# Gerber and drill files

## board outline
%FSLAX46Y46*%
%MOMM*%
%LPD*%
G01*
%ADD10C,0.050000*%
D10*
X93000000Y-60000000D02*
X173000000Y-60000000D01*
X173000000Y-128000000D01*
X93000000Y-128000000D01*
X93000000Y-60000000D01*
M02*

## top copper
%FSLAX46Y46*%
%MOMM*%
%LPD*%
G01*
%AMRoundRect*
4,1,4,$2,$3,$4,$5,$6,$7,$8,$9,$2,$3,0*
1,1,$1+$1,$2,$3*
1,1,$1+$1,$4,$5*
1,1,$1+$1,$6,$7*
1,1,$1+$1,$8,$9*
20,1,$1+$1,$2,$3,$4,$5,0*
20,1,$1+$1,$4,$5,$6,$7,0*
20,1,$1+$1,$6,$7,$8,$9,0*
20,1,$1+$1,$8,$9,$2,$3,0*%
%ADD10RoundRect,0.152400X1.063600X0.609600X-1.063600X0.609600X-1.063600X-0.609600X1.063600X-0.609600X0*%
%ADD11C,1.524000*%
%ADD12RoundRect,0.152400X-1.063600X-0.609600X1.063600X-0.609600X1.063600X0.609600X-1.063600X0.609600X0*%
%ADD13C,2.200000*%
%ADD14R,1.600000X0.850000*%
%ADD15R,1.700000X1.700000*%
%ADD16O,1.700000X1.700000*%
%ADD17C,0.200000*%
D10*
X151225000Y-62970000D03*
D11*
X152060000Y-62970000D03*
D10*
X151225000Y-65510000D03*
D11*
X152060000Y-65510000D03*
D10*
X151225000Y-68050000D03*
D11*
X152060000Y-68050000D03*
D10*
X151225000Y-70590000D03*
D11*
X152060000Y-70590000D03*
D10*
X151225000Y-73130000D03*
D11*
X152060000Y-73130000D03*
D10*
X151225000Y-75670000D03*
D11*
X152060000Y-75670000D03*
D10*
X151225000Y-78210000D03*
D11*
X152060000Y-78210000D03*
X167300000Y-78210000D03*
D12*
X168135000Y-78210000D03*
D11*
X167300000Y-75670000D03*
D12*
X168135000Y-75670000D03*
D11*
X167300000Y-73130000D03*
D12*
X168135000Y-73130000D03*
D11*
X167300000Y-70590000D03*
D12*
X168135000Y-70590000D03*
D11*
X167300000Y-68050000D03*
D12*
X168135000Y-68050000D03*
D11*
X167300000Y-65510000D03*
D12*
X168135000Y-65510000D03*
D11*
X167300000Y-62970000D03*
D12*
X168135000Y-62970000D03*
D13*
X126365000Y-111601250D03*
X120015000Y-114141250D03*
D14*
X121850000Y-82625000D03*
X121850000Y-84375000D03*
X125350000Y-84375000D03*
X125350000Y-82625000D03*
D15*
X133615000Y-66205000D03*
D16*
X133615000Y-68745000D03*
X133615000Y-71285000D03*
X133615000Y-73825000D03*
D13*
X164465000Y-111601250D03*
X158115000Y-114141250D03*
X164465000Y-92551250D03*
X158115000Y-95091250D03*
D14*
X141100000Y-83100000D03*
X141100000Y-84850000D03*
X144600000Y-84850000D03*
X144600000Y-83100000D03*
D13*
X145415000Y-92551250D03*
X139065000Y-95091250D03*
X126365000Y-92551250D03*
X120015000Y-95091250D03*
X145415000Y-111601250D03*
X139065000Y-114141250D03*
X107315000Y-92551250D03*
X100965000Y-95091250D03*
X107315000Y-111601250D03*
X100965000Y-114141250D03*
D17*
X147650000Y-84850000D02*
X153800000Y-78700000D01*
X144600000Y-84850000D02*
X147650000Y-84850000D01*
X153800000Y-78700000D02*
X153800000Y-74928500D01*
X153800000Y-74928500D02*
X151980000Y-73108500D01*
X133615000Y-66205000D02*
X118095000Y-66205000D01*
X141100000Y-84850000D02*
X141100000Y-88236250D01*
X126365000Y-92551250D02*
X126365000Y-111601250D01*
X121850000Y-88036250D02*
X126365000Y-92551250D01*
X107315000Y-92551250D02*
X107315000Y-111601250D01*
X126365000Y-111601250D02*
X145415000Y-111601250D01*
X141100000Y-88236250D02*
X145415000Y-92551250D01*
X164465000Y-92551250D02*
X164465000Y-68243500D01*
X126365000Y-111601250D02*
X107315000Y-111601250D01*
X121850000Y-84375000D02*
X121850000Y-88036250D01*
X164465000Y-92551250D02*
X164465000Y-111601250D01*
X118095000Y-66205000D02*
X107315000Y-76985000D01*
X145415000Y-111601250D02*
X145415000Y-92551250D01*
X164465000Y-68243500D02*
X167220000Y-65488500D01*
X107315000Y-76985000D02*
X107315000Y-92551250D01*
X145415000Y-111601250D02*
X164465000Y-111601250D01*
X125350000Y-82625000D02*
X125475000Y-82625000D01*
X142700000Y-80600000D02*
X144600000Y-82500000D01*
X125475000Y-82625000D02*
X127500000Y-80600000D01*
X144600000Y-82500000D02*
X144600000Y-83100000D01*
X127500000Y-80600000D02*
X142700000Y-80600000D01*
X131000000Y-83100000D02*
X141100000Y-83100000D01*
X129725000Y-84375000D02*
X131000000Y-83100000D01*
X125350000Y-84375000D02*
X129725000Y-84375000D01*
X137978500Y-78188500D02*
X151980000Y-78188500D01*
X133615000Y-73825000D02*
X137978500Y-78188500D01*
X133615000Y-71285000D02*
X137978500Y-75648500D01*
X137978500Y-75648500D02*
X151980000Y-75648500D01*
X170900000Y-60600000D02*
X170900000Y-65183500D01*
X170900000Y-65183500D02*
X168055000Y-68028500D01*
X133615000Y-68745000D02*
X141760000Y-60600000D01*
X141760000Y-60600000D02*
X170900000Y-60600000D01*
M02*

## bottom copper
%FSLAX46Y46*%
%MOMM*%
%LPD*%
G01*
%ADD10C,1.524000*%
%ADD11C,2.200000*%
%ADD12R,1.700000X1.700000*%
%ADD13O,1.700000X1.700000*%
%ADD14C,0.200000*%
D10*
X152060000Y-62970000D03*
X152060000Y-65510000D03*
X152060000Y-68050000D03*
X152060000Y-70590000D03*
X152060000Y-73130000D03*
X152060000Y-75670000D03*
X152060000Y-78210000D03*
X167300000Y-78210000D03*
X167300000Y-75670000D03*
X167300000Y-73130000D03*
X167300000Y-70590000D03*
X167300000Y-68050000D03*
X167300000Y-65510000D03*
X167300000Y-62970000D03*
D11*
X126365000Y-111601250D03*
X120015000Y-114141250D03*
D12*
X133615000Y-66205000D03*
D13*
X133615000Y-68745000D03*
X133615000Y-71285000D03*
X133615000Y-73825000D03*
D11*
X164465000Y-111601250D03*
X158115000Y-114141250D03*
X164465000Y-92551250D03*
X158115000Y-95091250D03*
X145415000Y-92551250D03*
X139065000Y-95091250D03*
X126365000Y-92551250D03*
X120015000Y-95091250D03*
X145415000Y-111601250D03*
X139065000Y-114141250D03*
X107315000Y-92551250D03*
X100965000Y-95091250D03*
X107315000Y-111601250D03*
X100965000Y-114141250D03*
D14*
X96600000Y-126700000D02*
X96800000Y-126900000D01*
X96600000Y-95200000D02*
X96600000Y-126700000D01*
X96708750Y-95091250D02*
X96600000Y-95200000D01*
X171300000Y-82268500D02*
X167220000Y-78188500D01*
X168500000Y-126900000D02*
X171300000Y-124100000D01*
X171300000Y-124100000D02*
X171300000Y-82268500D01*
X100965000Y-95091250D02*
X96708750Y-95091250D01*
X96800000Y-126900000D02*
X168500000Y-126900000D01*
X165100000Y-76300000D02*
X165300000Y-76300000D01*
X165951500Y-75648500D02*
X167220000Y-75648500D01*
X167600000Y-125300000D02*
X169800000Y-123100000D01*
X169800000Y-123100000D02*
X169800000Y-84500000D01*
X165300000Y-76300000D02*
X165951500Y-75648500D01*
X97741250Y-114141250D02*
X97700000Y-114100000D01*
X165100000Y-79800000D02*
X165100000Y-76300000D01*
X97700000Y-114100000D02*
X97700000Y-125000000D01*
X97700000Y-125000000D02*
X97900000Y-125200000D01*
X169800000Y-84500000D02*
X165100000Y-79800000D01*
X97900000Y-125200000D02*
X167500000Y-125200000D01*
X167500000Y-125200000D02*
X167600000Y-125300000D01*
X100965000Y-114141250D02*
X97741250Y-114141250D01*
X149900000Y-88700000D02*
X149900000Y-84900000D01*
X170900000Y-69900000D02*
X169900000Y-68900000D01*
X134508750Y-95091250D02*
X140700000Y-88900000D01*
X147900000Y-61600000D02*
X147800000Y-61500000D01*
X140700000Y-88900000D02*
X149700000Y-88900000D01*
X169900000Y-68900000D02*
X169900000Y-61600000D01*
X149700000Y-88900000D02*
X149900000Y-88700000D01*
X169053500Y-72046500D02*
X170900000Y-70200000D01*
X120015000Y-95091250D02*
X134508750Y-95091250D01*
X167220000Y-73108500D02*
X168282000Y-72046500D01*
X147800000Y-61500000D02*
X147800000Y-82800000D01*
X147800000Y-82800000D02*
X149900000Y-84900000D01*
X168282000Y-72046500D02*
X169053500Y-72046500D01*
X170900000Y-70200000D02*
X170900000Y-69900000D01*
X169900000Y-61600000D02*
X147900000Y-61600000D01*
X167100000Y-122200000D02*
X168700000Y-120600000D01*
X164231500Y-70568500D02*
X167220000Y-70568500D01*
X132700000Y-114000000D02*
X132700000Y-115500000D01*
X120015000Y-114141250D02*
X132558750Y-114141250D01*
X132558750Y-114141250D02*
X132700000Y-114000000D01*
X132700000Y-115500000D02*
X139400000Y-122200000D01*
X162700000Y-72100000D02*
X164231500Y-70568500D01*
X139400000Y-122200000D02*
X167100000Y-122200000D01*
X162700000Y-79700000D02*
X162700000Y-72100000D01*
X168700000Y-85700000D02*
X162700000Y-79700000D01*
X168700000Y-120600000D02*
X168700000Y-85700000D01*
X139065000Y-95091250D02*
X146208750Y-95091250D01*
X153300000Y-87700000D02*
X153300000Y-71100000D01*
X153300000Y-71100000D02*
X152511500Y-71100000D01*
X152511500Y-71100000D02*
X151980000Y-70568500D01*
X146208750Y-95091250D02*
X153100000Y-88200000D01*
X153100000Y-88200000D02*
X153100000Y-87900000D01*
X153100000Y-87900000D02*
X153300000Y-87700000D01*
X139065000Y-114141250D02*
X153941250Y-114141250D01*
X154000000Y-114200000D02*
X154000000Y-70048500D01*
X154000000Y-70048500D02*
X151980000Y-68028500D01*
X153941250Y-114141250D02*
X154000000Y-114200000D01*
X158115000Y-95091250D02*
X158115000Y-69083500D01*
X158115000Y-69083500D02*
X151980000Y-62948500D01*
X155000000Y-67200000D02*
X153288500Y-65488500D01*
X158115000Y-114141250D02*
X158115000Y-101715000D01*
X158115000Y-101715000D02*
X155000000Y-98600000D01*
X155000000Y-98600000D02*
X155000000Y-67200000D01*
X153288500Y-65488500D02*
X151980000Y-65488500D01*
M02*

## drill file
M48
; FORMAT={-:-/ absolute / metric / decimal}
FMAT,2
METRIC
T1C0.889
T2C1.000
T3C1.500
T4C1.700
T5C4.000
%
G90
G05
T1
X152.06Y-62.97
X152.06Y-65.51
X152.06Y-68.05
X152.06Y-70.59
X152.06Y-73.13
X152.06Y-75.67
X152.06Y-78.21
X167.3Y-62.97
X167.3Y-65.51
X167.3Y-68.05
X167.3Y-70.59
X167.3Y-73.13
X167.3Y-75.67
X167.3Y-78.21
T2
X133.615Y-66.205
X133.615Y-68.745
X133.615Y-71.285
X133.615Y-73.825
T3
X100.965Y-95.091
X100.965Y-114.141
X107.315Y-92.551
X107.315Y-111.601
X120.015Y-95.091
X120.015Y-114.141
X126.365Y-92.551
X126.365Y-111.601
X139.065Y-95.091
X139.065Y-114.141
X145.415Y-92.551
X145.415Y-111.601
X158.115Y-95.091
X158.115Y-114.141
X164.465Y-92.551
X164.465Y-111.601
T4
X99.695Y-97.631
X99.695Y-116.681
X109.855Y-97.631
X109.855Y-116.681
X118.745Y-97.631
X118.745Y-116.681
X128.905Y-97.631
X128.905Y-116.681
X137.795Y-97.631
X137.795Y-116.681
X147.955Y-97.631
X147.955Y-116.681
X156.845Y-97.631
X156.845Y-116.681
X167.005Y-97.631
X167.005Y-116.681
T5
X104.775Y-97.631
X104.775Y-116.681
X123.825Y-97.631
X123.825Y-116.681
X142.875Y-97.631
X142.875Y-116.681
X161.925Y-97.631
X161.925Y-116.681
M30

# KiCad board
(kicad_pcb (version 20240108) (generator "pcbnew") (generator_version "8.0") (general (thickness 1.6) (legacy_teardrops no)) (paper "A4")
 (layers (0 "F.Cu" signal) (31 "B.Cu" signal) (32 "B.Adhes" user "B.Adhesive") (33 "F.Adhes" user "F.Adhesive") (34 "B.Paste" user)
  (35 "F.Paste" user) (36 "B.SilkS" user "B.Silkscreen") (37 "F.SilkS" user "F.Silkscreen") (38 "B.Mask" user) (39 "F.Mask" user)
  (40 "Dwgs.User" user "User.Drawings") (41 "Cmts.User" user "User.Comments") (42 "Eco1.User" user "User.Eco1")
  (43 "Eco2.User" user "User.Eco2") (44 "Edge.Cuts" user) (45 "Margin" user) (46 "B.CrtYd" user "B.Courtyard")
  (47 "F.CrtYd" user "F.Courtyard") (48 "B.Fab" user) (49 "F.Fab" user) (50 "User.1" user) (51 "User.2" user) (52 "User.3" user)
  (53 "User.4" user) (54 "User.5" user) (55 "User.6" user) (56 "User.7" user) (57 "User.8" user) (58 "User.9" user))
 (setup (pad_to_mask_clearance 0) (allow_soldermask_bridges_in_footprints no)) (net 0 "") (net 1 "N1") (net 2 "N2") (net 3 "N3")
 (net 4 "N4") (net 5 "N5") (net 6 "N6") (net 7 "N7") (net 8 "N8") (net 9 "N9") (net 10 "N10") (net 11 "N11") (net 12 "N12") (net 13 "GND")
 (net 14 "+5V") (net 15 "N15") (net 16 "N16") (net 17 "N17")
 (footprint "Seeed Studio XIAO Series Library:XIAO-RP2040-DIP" (layer "F.Cu") (at 159.68 70.59)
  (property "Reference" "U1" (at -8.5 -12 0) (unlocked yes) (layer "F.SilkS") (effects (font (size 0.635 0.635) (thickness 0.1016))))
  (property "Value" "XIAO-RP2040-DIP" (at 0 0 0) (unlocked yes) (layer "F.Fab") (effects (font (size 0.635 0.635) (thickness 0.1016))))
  (pad "1" smd roundrect (at -8.455 -7.62 180) (size 2.432 1.524) (layers "F.Cu" "F.Mask") (roundrect_rratio 0.1) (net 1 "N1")
   (thermal_bridge_angle 45))
  (pad "1" thru_hole circle (at -7.62 -7.62 180) (size 1.524 1.524) (drill 0.889) (layers "*.Cu" "*.Mask") (remove_unused_layers no)
   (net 1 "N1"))
  (pad "2" smd roundrect (at -8.455 -5.08 180) (size 2.432 1.524) (layers "F.Cu" "F.Mask") (roundrect_rratio 0.1) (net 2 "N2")
   (thermal_bridge_angle 45))
  (pad "2" thru_hole circle (at -7.62 -5.08 180) (size 1.524 1.524) (drill 0.889) (layers "*.Cu" "*.Mask") (remove_unused_layers no)
   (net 2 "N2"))
  (pad "3" smd roundrect (at -8.455 -2.54 180) (size 2.432 1.524) (layers "F.Cu" "F.Mask") (roundrect_rratio 0.1) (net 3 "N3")
   (thermal_bridge_angle 45))
  (pad "3" thru_hole circle (at -7.62 -2.54 180) (size 1.524 1.524) (drill 0.889) (layers "*.Cu" "*.Mask") (remove_unused_layers no)
   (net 3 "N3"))
  (pad "4" smd roundrect (at -8.455 0 180) (size 2.432 1.524) (layers "F.Cu" "F.Mask") (roundrect_rratio 0.1) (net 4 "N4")
   (thermal_bridge_angle 45))
  (pad "4" thru_hole circle (at -7.62 0 180) (size 1.524 1.524) (drill 0.889) (layers "*.Cu" "*.Mask") (remove_unused_layers no)
   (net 4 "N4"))
  (pad "5" smd roundrect (at -8.455 2.54 180) (size 2.432 1.524) (layers "F.Cu" "F.Mask") (roundrect_rratio 0.1) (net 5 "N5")
   (thermal_bridge_angle 45))
  (pad "5" thru_hole circle (at -7.62 2.54 180) (size 1.524 1.524) (drill 0.889) (layers "*.Cu" "*.Mask") (remove_unused_layers no)
   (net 5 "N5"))
  (pad "6" smd roundrect (at -8.455 5.08 180) (size 2.432 1.524) (layers "F.Cu" "F.Mask") (roundrect_rratio 0.1) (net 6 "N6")
   (thermal_bridge_angle 45))
  (pad "6" thru_hole circle (at -7.62 5.08 180) (size 1.524 1.524) (drill 0.889) (layers "*.Cu" "*.Mask") (remove_unused_layers no)
   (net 6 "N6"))
  (pad "7" smd roundrect (at -8.455 7.62 180) (size 2.432 1.524) (layers "F.Cu" "F.Mask") (roundrect_rratio 0.1) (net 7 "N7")
   (thermal_bridge_angle 45))
  (pad "7" thru_hole circle (at -7.62 7.62 180) (size 1.524 1.524) (drill 0.889) (layers "*.Cu" "*.Mask") (remove_unused_layers no)
   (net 7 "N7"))
  (pad "8" thru_hole circle (at 7.62 7.62) (size 1.524 1.524) (drill 0.889) (layers "*.Cu" "*.Mask") (remove_unused_layers no) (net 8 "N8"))
  (pad "8" smd roundrect (at 8.455 7.62) (size 2.432 1.524) (layers "F.Cu" "F.Mask") (roundrect_rratio 0.1) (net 8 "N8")
   (thermal_bridge_angle 45))
  (pad "9" thru_hole circle (at 7.62 5.08) (size 1.524 1.524) (drill 0.889) (layers "*.Cu" "*.Mask") (remove_unused_layers no) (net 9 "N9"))
  (pad "9" smd roundrect (at 8.455 5.08) (size 2.432 1.524) (layers "F.Cu" "F.Mask") (roundrect_rratio 0.1) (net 9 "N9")
   (thermal_bridge_angle 45))
  (pad "10" thru_hole circle (at 7.62 2.54) (size 1.524 1.524) (drill 0.889) (layers "*.Cu" "*.Mask") (remove_unused_layers no)
   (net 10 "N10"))
  (pad "10" smd roundrect (at 8.455 2.54) (size 2.432 1.524) (layers "F.Cu" "F.Mask") (roundrect_rratio 0.1) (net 10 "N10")
   (thermal_bridge_angle 45))
  (pad "11" thru_hole circle (at 7.62 0) (size 1.524 1.524) (drill 0.889) (layers "*.Cu" "*.Mask") (remove_unused_layers no) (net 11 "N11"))
  (pad "11" smd roundrect (at 8.455 0) (size 2.432 1.524) (layers "F.Cu" "F.Mask") (roundrect_rratio 0.1) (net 11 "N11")
   (thermal_bridge_angle 45))
  (pad "12" thru_hole circle (at 7.62 -2.54) (size 1.524 1.524) (drill 0.889) (layers "*.Cu" "*.Mask") (remove_unused_layers no)
   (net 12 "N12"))
  (pad "12" smd roundrect (at 8.455 -2.54) (size 2.432 1.524) (layers "F.Cu" "F.Mask") (roundrect_rratio 0.1) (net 12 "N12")
   (thermal_bridge_angle 45))
  (pad "13" thru_hole circle (at 7.62 -5.08) (size 1.524 1.524) (drill 0.889) (layers "*.Cu" "*.Mask") (remove_unused_layers no)
   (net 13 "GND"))
  (pad "13" smd roundrect (at 8.455 -5.08) (size 2.432 1.524) (layers "F.Cu" "F.Mask") (roundrect_rratio 0.1) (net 13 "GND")
   (thermal_bridge_angle 45))
  (pad "14" thru_hole circle (at 7.62 -7.62) (size 1.524 1.524) (drill 0.889) (layers "*.Cu" "*.Mask") (remove_unused_layers no)
   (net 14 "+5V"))
  (pad "14" smd roundrect (at 8.455 -7.62) (size 2.432 1.524) (layers "F.Cu" "F.Mask") (roundrect_rratio 0.1) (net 14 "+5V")
   (thermal_bridge_angle 45)))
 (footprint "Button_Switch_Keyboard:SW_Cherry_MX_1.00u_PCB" (layer "F.Cu") (at 126.365 111.60125)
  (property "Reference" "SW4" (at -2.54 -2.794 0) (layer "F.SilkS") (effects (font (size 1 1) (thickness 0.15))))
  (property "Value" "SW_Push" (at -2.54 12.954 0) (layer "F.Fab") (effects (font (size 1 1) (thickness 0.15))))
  (pad "" np_thru_hole circle (at -7.62 5.08) (size 1.7 1.7) (drill 1.7) (layers "*.Cu" "*.Mask"))
  (pad "" np_thru_hole circle (at -2.54 5.08) (size 4 4) (drill 4) (layers "*.Cu" "*.Mask"))
  (pad "" np_thru_hole circle (at 2.54 5.08) (size 1.7 1.7) (drill 1.7) (layers "*.Cu" "*.Mask"))
  (pad "1" thru_hole circle (at 0 0) (size 2.2 2.2) (drill 1.5) (layers "*.Cu" "*.Mask") (remove_unused_layers no) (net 13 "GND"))
  (pad "2" thru_hole circle (at -6.35 2.54) (size 2.2 2.2) (drill 1.5) (layers "*.Cu" "*.Mask") (remove_unused_layers no) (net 11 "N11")))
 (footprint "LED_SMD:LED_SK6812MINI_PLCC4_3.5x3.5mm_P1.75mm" (layer "F.Cu") (at 123.6 83.5)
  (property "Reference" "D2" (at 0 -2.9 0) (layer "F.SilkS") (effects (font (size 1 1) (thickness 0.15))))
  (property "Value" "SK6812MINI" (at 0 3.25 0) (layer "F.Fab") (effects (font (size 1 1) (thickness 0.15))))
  (pad "1" smd rect (at -1.75 -0.875) (size 1.6 0.85) (layers "F.Cu" "F.Paste" "F.Mask") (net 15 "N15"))
  (pad "2" smd rect (at -1.75 0.875) (size 1.6 0.85) (layers "F.Cu" "F.Paste" "F.Mask") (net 13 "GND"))
  (pad "3" smd rect (at 1.75 0.875) (size 1.6 0.85) (layers "F.Cu" "F.Paste" "F.Mask") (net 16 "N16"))
  (pad "4" smd rect (at 1.75 -0.875) (size 1.6 0.85) (layers "F.Cu" "F.Paste" "F.Mask") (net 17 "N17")))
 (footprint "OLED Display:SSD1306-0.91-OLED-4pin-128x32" (layer "F.Cu") (at 97.115 64.015)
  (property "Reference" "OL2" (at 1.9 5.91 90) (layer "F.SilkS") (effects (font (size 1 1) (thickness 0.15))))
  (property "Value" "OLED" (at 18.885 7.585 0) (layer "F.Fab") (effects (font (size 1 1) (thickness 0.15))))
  (pad "1" thru_hole rect (at 36.5 2.19) (size 1.7 1.7) (drill 1) (layers "*.Cu" "*.Mask") (remove_unused_layers no) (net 13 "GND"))
  (pad "2" thru_hole oval (at 36.5 4.73) (size 1.7 1.7) (drill 1) (layers "*.Cu" "*.Mask") (remove_unused_layers no) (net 12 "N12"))
  (pad "3" thru_hole oval (at 36.5 7.27) (size 1.7 1.7) (drill 1) (layers "*.Cu" "*.Mask") (remove_unused_layers no) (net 6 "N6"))
  (pad "4" thru_hole oval (at 36.5 9.81) (size 1.7 1.7) (drill 1) (layers "*.Cu" "*.Mask") (remove_unused_layers no) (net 7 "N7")))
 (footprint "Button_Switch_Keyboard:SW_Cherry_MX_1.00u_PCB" (layer "F.Cu") (at 164.465 111.60125)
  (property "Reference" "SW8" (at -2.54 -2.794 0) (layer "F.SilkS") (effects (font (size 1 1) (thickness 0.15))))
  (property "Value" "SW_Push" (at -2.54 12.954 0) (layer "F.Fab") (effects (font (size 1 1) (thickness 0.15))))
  (pad "" np_thru_hole circle (at -7.62 5.08) (size 1.7 1.7) (drill 1.7) (layers "*.Cu" "*.Mask"))
  (pad "" np_thru_hole circle (at -2.54 5.08) (size 4 4) (drill 4) (layers "*.Cu" "*.Mask"))
  (pad "" np_thru_hole circle (at 2.54 5.08) (size 1.7 1.7) (drill 1.7) (layers "*.Cu" "*.Mask"))
  (pad "1" thru_hole circle (at 0 0) (size 2.2 2.2) (drill 1.5) (layers "*.Cu" "*.Mask") (remove_unused_layers no) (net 13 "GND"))
  (pad "2" thru_hole circle (at -6.35 2.54) (size 2.2 2.2) (drill 1.5) (layers "*.Cu" "*.Mask") (remove_unused_layers no) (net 2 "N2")))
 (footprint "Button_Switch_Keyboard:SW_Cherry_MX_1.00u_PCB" (layer "F.Cu") (at 164.465 92.55125)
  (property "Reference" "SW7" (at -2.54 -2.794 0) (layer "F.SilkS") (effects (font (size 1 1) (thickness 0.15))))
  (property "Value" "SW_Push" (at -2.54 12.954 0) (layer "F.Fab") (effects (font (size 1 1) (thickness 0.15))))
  (pad "" np_thru_hole circle (at -7.62 5.08) (size 1.7 1.7) (drill 1.7) (layers "*.Cu" "*.Mask"))
  (pad "" np_thru_hole circle (at -2.54 5.08) (size 4 4) (drill 4) (layers "*.Cu" "*.Mask"))
  (pad "" np_thru_hole circle (at 2.54 5.08) (size 1.7 1.7) (drill 1.7) (layers "*.Cu" "*.Mask"))
  (pad "1" thru_hole circle (at 0 0) (size 2.2 2.2) (drill 1.5) (layers "*.Cu" "*.Mask") (remove_unused_layers no) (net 13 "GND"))
  (pad "2" thru_hole circle (at -6.35 2.54) (size 2.2 2.2) (drill 1.5) (layers "*.Cu" "*.Mask") (remove_unused_layers no) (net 1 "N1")))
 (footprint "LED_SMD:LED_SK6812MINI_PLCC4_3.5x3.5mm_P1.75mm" (layer "F.Cu") (at 142.85 83.975)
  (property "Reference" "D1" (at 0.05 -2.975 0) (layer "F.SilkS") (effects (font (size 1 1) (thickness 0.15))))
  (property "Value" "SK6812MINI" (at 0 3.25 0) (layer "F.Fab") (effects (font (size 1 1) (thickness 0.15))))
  (pad "1" smd rect (at -1.75 -0.875) (size 1.6 0.85) (layers "F.Cu" "F.Paste" "F.Mask") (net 16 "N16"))
  (pad "2" smd rect (at -1.75 0.875) (size 1.6 0.85) (layers "F.Cu" "F.Paste" "F.Mask") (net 13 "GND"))
  (pad "3" smd rect (at 1.75 0.875) (size 1.6 0.85) (layers "F.Cu" "F.Paste" "F.Mask") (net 5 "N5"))
  (pad "4" smd rect (at 1.75 -0.875) (size 1.6 0.85) (layers "F.Cu" "F.Paste" "F.Mask") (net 17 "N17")))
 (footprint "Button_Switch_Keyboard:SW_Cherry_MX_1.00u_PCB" (layer "F.Cu") (at 145.415 92.55125)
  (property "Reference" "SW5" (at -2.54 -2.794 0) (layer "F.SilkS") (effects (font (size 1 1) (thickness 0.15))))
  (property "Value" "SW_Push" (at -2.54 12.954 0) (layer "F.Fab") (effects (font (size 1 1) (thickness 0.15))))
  (pad "" np_thru_hole circle (at -7.62 5.08) (size 1.7 1.7) (drill 1.7) (layers "*.Cu" "*.Mask"))
  (pad "" np_thru_hole circle (at -2.54 5.08) (size 4 4) (drill 4) (layers "*.Cu" "*.Mask"))
  (pad "" np_thru_hole circle (at 2.54 5.08) (size 1.7 1.7) (drill 1.7) (layers "*.Cu" "*.Mask"))
  (pad "1" thru_hole circle (at 0 0) (size 2.2 2.2) (drill 1.5) (layers "*.Cu" "*.Mask") (remove_unused_layers no) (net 13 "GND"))
  (pad "2" thru_hole circle (at -6.35 2.54) (size 2.2 2.2) (drill 1.5) (layers "*.Cu" "*.Mask") (remove_unused_layers no) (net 4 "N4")))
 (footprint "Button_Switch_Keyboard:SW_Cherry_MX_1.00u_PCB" (layer "F.Cu") (at 126.365 92.55125)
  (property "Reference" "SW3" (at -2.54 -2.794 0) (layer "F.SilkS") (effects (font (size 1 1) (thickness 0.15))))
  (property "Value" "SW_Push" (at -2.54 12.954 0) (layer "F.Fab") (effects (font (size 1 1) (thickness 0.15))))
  (pad "" np_thru_hole circle (at -7.62 5.08) (size 1.7 1.7) (drill 1.7) (layers "*.Cu" "*.Mask"))
  (pad "" np_thru_hole circle (at -2.54 5.08) (size 4 4) (drill 4) (layers "*.Cu" "*.Mask"))
  (pad "" np_thru_hole circle (at 2.54 5.08) (size 1.7 1.7) (drill 1.7) (layers "*.Cu" "*.Mask"))
  (pad "1" thru_hole circle (at 0 0) (size 2.2 2.2) (drill 1.5) (layers "*.Cu" "*.Mask") (remove_unused_layers no) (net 13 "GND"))
  (pad "2" thru_hole circle (at -6.35 2.54) (size 2.2 2.2) (drill 1.5) (layers "*.Cu" "*.Mask") (remove_unused_layers no) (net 10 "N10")))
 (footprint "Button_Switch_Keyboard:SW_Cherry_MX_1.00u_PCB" (layer "F.Cu") (at 145.415 111.60125)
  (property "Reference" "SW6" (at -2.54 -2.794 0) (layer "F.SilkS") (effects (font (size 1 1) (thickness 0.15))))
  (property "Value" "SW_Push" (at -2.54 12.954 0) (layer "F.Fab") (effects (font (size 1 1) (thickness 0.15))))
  (pad "" np_thru_hole circle (at -7.62 5.08) (size 1.7 1.7) (drill 1.7) (layers "*.Cu" "*.Mask"))
  (pad "" np_thru_hole circle (at -2.54 5.08) (size 4 4) (drill 4) (layers "*.Cu" "*.Mask"))
  (pad "" np_thru_hole circle (at 2.54 5.08) (size 1.7 1.7) (drill 1.7) (layers "*.Cu" "*.Mask"))
  (pad "1" thru_hole circle (at 0 0) (size 2.2 2.2) (drill 1.5) (layers "*.Cu" "*.Mask") (remove_unused_layers no) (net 13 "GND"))
  (pad "2" thru_hole circle (at -6.35 2.54) (size 2.2 2.2) (drill 1.5) (layers "*.Cu" "*.Mask") (remove_unused_layers no) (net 3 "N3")))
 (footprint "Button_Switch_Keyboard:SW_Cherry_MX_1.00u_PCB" (layer "F.Cu") (at 107.315 92.55125)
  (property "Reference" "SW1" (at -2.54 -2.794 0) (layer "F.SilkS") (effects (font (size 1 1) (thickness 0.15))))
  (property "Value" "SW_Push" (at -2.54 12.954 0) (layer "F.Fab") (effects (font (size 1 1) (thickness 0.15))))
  (pad "" np_thru_hole circle (at -7.62 5.08) (size 1.7 1.7) (drill 1.7) (layers "*.Cu" "*.Mask"))
  (pad "" np_thru_hole circle (at -2.54 5.08) (size 4 4) (drill 4) (layers "*.Cu" "*.Mask"))
  (pad "" np_thru_hole circle (at 2.54 5.08) (size 1.7 1.7) (drill 1.7) (layers "*.Cu" "*.Mask"))
  (pad "1" thru_hole circle (at 0 0) (size 2.2 2.2) (drill 1.5) (layers "*.Cu" "*.Mask") (remove_unused_layers no) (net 13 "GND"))
  (pad "2" thru_hole circle (at -6.35 2.54) (size 2.2 2.2) (drill 1.5) (layers "*.Cu" "*.Mask") (remove_unused_layers no) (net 8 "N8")))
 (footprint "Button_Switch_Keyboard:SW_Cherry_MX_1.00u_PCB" (layer "F.Cu") (at 107.315 111.60125)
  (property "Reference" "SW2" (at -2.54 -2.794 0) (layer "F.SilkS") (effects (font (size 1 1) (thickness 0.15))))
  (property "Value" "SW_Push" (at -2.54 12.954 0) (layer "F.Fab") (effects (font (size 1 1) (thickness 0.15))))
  (pad "" np_thru_hole circle (at -7.62 5.08) (size 1.7 1.7) (drill 1.7) (layers "*.Cu" "*.Mask"))
  (pad "" np_thru_hole circle (at -2.54 5.08) (size 4 4) (drill 4) (layers "*.Cu" "*.Mask"))
  (pad "" np_thru_hole circle (at 2.54 5.08) (size 1.7 1.7) (drill 1.7) (layers "*.Cu" "*.Mask"))
  (pad "1" thru_hole circle (at 0 0) (size 2.2 2.2) (drill 1.5) (layers "*.Cu" "*.Mask") (remove_unused_layers no) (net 13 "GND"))
  (pad "2" thru_hole circle (at -6.35 2.54) (size 2.2 2.2) (drill 1.5) (layers "*.Cu" "*.Mask") (remove_unused_layers no) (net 9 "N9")))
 (gr_rect (start 93 60) (end 173 128) (stroke (width 0.05) (type default)) (fill none) (layer "Edge.Cuts"))
 (segment (start 147.65 84.85) (end 153.8 78.7) (width 0.2) (layer "F.Cu") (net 5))
 (segment (start 144.6 84.85) (end 147.65 84.85) (width 0.2) (layer "F.Cu") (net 5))
 (segment (start 153.8 78.7) (end 153.8 74.9285) (width 0.2) (layer "F.Cu") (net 5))
 (segment (start 153.8 74.9285) (end 151.98 73.1085) (width 0.2) (layer "F.Cu") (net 5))
 (segment (start 133.615 66.205) (end 118.095 66.205) (width 0.2) (layer "F.Cu") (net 13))
 (segment (start 141.1 84.85) (end 141.1 88.23625) (width 0.2) (layer "F.Cu") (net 13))
 (segment (start 126.365 92.55125) (end 126.365 111.60125) (width 0.2) (layer "F.Cu") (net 13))
 (segment (start 121.85 88.03625) (end 126.365 92.55125) (width 0.2) (layer "F.Cu") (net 13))
 (segment (start 107.315 92.55125) (end 107.315 111.60125) (width 0.2) (layer "F.Cu") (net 13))
 (segment (start 126.365 111.60125) (end 145.415 111.60125) (width 0.2) (layer "F.Cu") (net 13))
 (segment (start 141.1 88.23625) (end 145.415 92.55125) (width 0.2) (layer "F.Cu") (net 13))
 (segment (start 164.465 92.55125) (end 164.465 68.2435) (width 0.2) (layer "F.Cu") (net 13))
 (segment (start 126.365 111.60125) (end 107.315 111.60125) (width 0.2) (layer "F.Cu") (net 13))
 (segment (start 121.85 84.375) (end 121.85 88.03625) (width 0.2) (layer "F.Cu") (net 13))
 (segment (start 164.465 92.55125) (end 164.465 111.60125) (width 0.2) (layer "F.Cu") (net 13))
 (segment (start 118.095 66.205) (end 107.315 76.985) (width 0.2) (layer "F.Cu") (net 13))
 (segment (start 145.415 111.60125) (end 145.415 92.55125) (width 0.2) (layer "F.Cu") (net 13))
 (segment (start 164.465 68.2435) (end 167.22 65.4885) (width 0.2) (layer "F.Cu") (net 13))
 (segment (start 107.315 76.985) (end 107.315 92.55125) (width 0.2) (layer "F.Cu") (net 13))
 (segment (start 145.415 111.60125) (end 164.465 111.60125) (width 0.2) (layer "F.Cu") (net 13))
 (segment (start 125.35 82.625) (end 125.475 82.625) (width 0.2) (layer "F.Cu") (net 17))
 (segment (start 142.7 80.6) (end 144.6 82.5) (width 0.2) (layer "F.Cu") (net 17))
 (segment (start 125.475 82.625) (end 127.5 80.6) (width 0.2) (layer "F.Cu") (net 17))
 (segment (start 144.6 82.5) (end 144.6 83.1) (width 0.2) (layer "F.Cu") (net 17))
 (segment (start 127.5 80.6) (end 142.7 80.6) (width 0.2) (layer "F.Cu") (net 17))
 (segment (start 131 83.1) (end 141.1 83.1) (width 0.2) (layer "F.Cu") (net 16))
 (segment (start 129.725 84.375) (end 131 83.1) (width 0.2) (layer "F.Cu") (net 16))
 (segment (start 125.35 84.375) (end 129.725 84.375) (width 0.2) (layer "F.Cu") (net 16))
 (segment (start 137.9785 78.1885) (end 151.98 78.1885) (width 0.2) (layer "F.Cu") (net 7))
 (segment (start 133.615 73.825) (end 137.9785 78.1885) (width 0.2) (layer "F.Cu") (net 7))
 (segment (start 133.615 71.285) (end 137.9785 75.6485) (width 0.2) (layer "F.Cu") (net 6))
 (segment (start 137.9785 75.6485) (end 151.98 75.6485) (width 0.2) (layer "F.Cu") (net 6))
 (segment (start 170.9 60.6) (end 170.9 65.1835) (width 0.2) (layer "F.Cu") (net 12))
 (segment (start 170.9 65.1835) (end 168.055 68.0285) (width 0.2) (layer "F.Cu") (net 12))
 (segment (start 133.615 68.745) (end 141.76 60.6) (width 0.2) (layer "F.Cu") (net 12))
 (segment (start 141.76 60.6) (end 170.9 60.6) (width 0.2) (layer "F.Cu") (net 12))
 (segment (start 96.6 126.7) (end 96.8 126.9) (width 0.2) (layer "B.Cu") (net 8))
 (segment (start 96.6 95.2) (end 96.6 126.7) (width 0.2) (layer "B.Cu") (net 8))
 (segment (start 96.70875 95.09125) (end 96.6 95.2) (width 0.2) (layer "B.Cu") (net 8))
 (segment (start 171.3 82.2685) (end 167.22 78.1885) (width 0.2) (layer "B.Cu") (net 8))
 (segment (start 168.5 126.9) (end 171.3 124.1) (width 0.2) (layer "B.Cu") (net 8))
 (segment (start 171.3 124.1) (end 171.3 82.2685) (width 0.2) (layer "B.Cu") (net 8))
 (segment (start 100.965 95.09125) (end 96.70875 95.09125) (width 0.2) (layer "B.Cu") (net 8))
 (segment (start 96.8 126.9) (end 168.5 126.9) (width 0.2) (layer "B.Cu") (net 8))
 (segment (start 165.1 76.3) (end 165.3 76.3) (width 0.2) (layer "B.Cu") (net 9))
 (segment (start 165.9515 75.6485) (end 167.22 75.6485) (width 0.2) (layer "B.Cu") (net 9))
 (segment (start 167.6 125.3) (end 169.8 123.1) (width 0.2) (layer "B.Cu") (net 9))
 (segment (start 169.8 123.1) (end 169.8 84.5) (width 0.2) (layer "B.Cu") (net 9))
 (segment (start 165.3 76.3) (end 165.9515 75.6485) (width 0.2) (layer "B.Cu") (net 9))
 (segment (start 97.74125 114.14125) (end 97.7 114.1) (width 0.2) (layer "B.Cu") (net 9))
 (segment (start 165.1 79.8) (end 165.1 76.3) (width 0.2) (layer "B.Cu") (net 9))
 (segment (start 97.7 114.1) (end 97.7 125) (width 0.2) (layer "B.Cu") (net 9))
 (segment (start 97.7 125) (end 97.9 125.2) (width 0.2) (layer "B.Cu") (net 9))
 (segment (start 169.8 84.5) (end 165.1 79.8) (width 0.2) (layer "B.Cu") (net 9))
 (segment (start 97.9 125.2) (end 167.5 125.2) (width 0.2) (layer "B.Cu") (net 9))
 (segment (start 167.5 125.2) (end 167.6 125.3) (width 0.2) (layer "B.Cu") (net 9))
 (segment (start 100.965 114.14125) (end 97.74125 114.14125) (width 0.2) (layer "B.Cu") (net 9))
 (segment (start 149.9 88.7) (end 149.9 84.9) (width 0.2) (layer "B.Cu") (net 10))
 (segment (start 170.9 69.9) (end 169.9 68.9) (width 0.2) (layer "B.Cu") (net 10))
 (segment (start 134.50875 95.09125) (end 140.7 88.9) (width 0.2) (layer "B.Cu") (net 10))
 (segment (start 147.9 61.6) (end 147.8 61.5) (width 0.2) (layer "B.Cu") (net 10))
 (segment (start 140.7 88.9) (end 149.7 88.9) (width 0.2) (layer "B.Cu") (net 10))
 (segment (start 169.9 68.9) (end 169.9 61.6) (width 0.2) (layer "B.Cu") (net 10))
 (segment (start 149.7 88.9) (end 149.9 88.7) (width 0.2) (layer "B.Cu") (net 10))
 (segment (start 169.0535 72.0465) (end 170.9 70.2) (width 0.2) (layer "B.Cu") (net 10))
 (segment (start 120.015 95.09125) (end 134.50875 95.09125) (width 0.2) (layer "B.Cu") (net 10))
 (segment (start 167.22 73.1085) (end 168.282 72.0465) (width 0.2) (layer "B.Cu") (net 10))
 (segment (start 147.8 61.5) (end 147.8 82.8) (width 0.2) (layer "B.Cu") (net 10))
 (segment (start 147.8 82.8) (end 149.9 84.9) (width 0.2) (layer "B.Cu") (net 10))
 (segment (start 168.282 72.0465) (end 169.0535 72.0465) (width 0.2) (layer "B.Cu") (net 10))
 (segment (start 170.9 70.2) (end 170.9 69.9) (width 0.2) (layer "B.Cu") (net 10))
 (segment (start 169.9 61.6) (end 147.9 61.6) (width 0.2) (layer "B.Cu") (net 10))
 (segment (start 167.1 122.2) (end 168.7 120.6) (width 0.2) (layer "B.Cu") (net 11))
 (segment (start 164.2315 70.5685) (end 167.22 70.5685) (width 0.2) (layer "B.Cu") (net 11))
 (segment (start 132.7 114) (end 132.7 115.5) (width 0.2) (layer "B.Cu") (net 11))
 (segment (start 120.015 114.14125) (end 132.55875 114.14125) (width 0.2) (layer "B.Cu") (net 11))
 (segment (start 132.55875 114.14125) (end 132.7 114) (width 0.2) (layer "B.Cu") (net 11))
 (segment (start 132.7 115.5) (end 139.4 122.2) (width 0.2) (layer "B.Cu") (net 11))
 (segment (start 162.7 72.1) (end 164.2315 70.5685) (width 0.2) (layer "B.Cu") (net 11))
 (segment (start 139.4 122.2) (end 167.1 122.2) (width 0.2) (layer "B.Cu") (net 11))
 (segment (start 162.7 79.7) (end 162.7 72.1) (width 0.2) (layer "B.Cu") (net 11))
 (segment (start 168.7 85.7) (end 162.7 79.7) (width 0.2) (layer "B.Cu") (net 11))
 (segment (start 168.7 120.6) (end 168.7 85.7) (width 0.2) (layer "B.Cu") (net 11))
 (segment (start 139.065 95.09125) (end 146.20875 95.09125) (width 0.2) (layer "B.Cu") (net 4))
 (segment (start 153.3 87.7) (end 153.3 71.1) (width 0.2) (layer "B.Cu") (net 4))
 (segment (start 153.3 71.1) (end 152.5115 71.1) (width 0.2) (layer "B.Cu") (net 4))
 (segment (start 152.5115 71.1) (end 151.98 70.5685) (width 0.2) (layer "B.Cu") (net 4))
 (segment (start 146.20875 95.09125) (end 153.1 88.2) (width 0.2) (layer "B.Cu") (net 4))
 (segment (start 153.1 88.2) (end 153.1 87.9) (width 0.2) (layer "B.Cu") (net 4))
 (segment (start 153.1 87.9) (end 153.3 87.7) (width 0.2) (layer "B.Cu") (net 4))
 (segment (start 139.065 114.14125) (end 153.94125 114.14125) (width 0.2) (layer "B.Cu") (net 3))
 (segment (start 154 114.2) (end 154 70.0485) (width 0.2) (layer "B.Cu") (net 3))
 (segment (start 154 70.0485) (end 151.98 68.0285) (width 0.2) (layer "B.Cu") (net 3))
 (segment (start 153.94125 114.14125) (end 154 114.2) (width 0.2) (layer "B.Cu") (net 3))
 (segment (start 158.115 95.09125) (end 158.115 69.0835) (width 0.2) (layer "B.Cu") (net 1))
 (segment (start 158.115 69.0835) (end 151.98 62.9485) (width 0.2) (layer "B.Cu") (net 1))
 (segment (start 155 67.2) (end 153.2885 65.4885) (width 0.2) (layer "B.Cu") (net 2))
 (segment (start 158.115 114.14125) (end 158.115 101.715) (width 0.2) (layer "B.Cu") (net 2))
 (segment (start 158.115 101.715) (end 155 98.6) (width 0.2) (layer "B.Cu") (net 2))
 (segment (start 155 98.6) (end 155 67.2) (width 0.2) (layer "B.Cu") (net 2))
 (segment (start 153.2885 65.4885) (end 151.98 65.4885) (width 0.2) (layer "B.Cu") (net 2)))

